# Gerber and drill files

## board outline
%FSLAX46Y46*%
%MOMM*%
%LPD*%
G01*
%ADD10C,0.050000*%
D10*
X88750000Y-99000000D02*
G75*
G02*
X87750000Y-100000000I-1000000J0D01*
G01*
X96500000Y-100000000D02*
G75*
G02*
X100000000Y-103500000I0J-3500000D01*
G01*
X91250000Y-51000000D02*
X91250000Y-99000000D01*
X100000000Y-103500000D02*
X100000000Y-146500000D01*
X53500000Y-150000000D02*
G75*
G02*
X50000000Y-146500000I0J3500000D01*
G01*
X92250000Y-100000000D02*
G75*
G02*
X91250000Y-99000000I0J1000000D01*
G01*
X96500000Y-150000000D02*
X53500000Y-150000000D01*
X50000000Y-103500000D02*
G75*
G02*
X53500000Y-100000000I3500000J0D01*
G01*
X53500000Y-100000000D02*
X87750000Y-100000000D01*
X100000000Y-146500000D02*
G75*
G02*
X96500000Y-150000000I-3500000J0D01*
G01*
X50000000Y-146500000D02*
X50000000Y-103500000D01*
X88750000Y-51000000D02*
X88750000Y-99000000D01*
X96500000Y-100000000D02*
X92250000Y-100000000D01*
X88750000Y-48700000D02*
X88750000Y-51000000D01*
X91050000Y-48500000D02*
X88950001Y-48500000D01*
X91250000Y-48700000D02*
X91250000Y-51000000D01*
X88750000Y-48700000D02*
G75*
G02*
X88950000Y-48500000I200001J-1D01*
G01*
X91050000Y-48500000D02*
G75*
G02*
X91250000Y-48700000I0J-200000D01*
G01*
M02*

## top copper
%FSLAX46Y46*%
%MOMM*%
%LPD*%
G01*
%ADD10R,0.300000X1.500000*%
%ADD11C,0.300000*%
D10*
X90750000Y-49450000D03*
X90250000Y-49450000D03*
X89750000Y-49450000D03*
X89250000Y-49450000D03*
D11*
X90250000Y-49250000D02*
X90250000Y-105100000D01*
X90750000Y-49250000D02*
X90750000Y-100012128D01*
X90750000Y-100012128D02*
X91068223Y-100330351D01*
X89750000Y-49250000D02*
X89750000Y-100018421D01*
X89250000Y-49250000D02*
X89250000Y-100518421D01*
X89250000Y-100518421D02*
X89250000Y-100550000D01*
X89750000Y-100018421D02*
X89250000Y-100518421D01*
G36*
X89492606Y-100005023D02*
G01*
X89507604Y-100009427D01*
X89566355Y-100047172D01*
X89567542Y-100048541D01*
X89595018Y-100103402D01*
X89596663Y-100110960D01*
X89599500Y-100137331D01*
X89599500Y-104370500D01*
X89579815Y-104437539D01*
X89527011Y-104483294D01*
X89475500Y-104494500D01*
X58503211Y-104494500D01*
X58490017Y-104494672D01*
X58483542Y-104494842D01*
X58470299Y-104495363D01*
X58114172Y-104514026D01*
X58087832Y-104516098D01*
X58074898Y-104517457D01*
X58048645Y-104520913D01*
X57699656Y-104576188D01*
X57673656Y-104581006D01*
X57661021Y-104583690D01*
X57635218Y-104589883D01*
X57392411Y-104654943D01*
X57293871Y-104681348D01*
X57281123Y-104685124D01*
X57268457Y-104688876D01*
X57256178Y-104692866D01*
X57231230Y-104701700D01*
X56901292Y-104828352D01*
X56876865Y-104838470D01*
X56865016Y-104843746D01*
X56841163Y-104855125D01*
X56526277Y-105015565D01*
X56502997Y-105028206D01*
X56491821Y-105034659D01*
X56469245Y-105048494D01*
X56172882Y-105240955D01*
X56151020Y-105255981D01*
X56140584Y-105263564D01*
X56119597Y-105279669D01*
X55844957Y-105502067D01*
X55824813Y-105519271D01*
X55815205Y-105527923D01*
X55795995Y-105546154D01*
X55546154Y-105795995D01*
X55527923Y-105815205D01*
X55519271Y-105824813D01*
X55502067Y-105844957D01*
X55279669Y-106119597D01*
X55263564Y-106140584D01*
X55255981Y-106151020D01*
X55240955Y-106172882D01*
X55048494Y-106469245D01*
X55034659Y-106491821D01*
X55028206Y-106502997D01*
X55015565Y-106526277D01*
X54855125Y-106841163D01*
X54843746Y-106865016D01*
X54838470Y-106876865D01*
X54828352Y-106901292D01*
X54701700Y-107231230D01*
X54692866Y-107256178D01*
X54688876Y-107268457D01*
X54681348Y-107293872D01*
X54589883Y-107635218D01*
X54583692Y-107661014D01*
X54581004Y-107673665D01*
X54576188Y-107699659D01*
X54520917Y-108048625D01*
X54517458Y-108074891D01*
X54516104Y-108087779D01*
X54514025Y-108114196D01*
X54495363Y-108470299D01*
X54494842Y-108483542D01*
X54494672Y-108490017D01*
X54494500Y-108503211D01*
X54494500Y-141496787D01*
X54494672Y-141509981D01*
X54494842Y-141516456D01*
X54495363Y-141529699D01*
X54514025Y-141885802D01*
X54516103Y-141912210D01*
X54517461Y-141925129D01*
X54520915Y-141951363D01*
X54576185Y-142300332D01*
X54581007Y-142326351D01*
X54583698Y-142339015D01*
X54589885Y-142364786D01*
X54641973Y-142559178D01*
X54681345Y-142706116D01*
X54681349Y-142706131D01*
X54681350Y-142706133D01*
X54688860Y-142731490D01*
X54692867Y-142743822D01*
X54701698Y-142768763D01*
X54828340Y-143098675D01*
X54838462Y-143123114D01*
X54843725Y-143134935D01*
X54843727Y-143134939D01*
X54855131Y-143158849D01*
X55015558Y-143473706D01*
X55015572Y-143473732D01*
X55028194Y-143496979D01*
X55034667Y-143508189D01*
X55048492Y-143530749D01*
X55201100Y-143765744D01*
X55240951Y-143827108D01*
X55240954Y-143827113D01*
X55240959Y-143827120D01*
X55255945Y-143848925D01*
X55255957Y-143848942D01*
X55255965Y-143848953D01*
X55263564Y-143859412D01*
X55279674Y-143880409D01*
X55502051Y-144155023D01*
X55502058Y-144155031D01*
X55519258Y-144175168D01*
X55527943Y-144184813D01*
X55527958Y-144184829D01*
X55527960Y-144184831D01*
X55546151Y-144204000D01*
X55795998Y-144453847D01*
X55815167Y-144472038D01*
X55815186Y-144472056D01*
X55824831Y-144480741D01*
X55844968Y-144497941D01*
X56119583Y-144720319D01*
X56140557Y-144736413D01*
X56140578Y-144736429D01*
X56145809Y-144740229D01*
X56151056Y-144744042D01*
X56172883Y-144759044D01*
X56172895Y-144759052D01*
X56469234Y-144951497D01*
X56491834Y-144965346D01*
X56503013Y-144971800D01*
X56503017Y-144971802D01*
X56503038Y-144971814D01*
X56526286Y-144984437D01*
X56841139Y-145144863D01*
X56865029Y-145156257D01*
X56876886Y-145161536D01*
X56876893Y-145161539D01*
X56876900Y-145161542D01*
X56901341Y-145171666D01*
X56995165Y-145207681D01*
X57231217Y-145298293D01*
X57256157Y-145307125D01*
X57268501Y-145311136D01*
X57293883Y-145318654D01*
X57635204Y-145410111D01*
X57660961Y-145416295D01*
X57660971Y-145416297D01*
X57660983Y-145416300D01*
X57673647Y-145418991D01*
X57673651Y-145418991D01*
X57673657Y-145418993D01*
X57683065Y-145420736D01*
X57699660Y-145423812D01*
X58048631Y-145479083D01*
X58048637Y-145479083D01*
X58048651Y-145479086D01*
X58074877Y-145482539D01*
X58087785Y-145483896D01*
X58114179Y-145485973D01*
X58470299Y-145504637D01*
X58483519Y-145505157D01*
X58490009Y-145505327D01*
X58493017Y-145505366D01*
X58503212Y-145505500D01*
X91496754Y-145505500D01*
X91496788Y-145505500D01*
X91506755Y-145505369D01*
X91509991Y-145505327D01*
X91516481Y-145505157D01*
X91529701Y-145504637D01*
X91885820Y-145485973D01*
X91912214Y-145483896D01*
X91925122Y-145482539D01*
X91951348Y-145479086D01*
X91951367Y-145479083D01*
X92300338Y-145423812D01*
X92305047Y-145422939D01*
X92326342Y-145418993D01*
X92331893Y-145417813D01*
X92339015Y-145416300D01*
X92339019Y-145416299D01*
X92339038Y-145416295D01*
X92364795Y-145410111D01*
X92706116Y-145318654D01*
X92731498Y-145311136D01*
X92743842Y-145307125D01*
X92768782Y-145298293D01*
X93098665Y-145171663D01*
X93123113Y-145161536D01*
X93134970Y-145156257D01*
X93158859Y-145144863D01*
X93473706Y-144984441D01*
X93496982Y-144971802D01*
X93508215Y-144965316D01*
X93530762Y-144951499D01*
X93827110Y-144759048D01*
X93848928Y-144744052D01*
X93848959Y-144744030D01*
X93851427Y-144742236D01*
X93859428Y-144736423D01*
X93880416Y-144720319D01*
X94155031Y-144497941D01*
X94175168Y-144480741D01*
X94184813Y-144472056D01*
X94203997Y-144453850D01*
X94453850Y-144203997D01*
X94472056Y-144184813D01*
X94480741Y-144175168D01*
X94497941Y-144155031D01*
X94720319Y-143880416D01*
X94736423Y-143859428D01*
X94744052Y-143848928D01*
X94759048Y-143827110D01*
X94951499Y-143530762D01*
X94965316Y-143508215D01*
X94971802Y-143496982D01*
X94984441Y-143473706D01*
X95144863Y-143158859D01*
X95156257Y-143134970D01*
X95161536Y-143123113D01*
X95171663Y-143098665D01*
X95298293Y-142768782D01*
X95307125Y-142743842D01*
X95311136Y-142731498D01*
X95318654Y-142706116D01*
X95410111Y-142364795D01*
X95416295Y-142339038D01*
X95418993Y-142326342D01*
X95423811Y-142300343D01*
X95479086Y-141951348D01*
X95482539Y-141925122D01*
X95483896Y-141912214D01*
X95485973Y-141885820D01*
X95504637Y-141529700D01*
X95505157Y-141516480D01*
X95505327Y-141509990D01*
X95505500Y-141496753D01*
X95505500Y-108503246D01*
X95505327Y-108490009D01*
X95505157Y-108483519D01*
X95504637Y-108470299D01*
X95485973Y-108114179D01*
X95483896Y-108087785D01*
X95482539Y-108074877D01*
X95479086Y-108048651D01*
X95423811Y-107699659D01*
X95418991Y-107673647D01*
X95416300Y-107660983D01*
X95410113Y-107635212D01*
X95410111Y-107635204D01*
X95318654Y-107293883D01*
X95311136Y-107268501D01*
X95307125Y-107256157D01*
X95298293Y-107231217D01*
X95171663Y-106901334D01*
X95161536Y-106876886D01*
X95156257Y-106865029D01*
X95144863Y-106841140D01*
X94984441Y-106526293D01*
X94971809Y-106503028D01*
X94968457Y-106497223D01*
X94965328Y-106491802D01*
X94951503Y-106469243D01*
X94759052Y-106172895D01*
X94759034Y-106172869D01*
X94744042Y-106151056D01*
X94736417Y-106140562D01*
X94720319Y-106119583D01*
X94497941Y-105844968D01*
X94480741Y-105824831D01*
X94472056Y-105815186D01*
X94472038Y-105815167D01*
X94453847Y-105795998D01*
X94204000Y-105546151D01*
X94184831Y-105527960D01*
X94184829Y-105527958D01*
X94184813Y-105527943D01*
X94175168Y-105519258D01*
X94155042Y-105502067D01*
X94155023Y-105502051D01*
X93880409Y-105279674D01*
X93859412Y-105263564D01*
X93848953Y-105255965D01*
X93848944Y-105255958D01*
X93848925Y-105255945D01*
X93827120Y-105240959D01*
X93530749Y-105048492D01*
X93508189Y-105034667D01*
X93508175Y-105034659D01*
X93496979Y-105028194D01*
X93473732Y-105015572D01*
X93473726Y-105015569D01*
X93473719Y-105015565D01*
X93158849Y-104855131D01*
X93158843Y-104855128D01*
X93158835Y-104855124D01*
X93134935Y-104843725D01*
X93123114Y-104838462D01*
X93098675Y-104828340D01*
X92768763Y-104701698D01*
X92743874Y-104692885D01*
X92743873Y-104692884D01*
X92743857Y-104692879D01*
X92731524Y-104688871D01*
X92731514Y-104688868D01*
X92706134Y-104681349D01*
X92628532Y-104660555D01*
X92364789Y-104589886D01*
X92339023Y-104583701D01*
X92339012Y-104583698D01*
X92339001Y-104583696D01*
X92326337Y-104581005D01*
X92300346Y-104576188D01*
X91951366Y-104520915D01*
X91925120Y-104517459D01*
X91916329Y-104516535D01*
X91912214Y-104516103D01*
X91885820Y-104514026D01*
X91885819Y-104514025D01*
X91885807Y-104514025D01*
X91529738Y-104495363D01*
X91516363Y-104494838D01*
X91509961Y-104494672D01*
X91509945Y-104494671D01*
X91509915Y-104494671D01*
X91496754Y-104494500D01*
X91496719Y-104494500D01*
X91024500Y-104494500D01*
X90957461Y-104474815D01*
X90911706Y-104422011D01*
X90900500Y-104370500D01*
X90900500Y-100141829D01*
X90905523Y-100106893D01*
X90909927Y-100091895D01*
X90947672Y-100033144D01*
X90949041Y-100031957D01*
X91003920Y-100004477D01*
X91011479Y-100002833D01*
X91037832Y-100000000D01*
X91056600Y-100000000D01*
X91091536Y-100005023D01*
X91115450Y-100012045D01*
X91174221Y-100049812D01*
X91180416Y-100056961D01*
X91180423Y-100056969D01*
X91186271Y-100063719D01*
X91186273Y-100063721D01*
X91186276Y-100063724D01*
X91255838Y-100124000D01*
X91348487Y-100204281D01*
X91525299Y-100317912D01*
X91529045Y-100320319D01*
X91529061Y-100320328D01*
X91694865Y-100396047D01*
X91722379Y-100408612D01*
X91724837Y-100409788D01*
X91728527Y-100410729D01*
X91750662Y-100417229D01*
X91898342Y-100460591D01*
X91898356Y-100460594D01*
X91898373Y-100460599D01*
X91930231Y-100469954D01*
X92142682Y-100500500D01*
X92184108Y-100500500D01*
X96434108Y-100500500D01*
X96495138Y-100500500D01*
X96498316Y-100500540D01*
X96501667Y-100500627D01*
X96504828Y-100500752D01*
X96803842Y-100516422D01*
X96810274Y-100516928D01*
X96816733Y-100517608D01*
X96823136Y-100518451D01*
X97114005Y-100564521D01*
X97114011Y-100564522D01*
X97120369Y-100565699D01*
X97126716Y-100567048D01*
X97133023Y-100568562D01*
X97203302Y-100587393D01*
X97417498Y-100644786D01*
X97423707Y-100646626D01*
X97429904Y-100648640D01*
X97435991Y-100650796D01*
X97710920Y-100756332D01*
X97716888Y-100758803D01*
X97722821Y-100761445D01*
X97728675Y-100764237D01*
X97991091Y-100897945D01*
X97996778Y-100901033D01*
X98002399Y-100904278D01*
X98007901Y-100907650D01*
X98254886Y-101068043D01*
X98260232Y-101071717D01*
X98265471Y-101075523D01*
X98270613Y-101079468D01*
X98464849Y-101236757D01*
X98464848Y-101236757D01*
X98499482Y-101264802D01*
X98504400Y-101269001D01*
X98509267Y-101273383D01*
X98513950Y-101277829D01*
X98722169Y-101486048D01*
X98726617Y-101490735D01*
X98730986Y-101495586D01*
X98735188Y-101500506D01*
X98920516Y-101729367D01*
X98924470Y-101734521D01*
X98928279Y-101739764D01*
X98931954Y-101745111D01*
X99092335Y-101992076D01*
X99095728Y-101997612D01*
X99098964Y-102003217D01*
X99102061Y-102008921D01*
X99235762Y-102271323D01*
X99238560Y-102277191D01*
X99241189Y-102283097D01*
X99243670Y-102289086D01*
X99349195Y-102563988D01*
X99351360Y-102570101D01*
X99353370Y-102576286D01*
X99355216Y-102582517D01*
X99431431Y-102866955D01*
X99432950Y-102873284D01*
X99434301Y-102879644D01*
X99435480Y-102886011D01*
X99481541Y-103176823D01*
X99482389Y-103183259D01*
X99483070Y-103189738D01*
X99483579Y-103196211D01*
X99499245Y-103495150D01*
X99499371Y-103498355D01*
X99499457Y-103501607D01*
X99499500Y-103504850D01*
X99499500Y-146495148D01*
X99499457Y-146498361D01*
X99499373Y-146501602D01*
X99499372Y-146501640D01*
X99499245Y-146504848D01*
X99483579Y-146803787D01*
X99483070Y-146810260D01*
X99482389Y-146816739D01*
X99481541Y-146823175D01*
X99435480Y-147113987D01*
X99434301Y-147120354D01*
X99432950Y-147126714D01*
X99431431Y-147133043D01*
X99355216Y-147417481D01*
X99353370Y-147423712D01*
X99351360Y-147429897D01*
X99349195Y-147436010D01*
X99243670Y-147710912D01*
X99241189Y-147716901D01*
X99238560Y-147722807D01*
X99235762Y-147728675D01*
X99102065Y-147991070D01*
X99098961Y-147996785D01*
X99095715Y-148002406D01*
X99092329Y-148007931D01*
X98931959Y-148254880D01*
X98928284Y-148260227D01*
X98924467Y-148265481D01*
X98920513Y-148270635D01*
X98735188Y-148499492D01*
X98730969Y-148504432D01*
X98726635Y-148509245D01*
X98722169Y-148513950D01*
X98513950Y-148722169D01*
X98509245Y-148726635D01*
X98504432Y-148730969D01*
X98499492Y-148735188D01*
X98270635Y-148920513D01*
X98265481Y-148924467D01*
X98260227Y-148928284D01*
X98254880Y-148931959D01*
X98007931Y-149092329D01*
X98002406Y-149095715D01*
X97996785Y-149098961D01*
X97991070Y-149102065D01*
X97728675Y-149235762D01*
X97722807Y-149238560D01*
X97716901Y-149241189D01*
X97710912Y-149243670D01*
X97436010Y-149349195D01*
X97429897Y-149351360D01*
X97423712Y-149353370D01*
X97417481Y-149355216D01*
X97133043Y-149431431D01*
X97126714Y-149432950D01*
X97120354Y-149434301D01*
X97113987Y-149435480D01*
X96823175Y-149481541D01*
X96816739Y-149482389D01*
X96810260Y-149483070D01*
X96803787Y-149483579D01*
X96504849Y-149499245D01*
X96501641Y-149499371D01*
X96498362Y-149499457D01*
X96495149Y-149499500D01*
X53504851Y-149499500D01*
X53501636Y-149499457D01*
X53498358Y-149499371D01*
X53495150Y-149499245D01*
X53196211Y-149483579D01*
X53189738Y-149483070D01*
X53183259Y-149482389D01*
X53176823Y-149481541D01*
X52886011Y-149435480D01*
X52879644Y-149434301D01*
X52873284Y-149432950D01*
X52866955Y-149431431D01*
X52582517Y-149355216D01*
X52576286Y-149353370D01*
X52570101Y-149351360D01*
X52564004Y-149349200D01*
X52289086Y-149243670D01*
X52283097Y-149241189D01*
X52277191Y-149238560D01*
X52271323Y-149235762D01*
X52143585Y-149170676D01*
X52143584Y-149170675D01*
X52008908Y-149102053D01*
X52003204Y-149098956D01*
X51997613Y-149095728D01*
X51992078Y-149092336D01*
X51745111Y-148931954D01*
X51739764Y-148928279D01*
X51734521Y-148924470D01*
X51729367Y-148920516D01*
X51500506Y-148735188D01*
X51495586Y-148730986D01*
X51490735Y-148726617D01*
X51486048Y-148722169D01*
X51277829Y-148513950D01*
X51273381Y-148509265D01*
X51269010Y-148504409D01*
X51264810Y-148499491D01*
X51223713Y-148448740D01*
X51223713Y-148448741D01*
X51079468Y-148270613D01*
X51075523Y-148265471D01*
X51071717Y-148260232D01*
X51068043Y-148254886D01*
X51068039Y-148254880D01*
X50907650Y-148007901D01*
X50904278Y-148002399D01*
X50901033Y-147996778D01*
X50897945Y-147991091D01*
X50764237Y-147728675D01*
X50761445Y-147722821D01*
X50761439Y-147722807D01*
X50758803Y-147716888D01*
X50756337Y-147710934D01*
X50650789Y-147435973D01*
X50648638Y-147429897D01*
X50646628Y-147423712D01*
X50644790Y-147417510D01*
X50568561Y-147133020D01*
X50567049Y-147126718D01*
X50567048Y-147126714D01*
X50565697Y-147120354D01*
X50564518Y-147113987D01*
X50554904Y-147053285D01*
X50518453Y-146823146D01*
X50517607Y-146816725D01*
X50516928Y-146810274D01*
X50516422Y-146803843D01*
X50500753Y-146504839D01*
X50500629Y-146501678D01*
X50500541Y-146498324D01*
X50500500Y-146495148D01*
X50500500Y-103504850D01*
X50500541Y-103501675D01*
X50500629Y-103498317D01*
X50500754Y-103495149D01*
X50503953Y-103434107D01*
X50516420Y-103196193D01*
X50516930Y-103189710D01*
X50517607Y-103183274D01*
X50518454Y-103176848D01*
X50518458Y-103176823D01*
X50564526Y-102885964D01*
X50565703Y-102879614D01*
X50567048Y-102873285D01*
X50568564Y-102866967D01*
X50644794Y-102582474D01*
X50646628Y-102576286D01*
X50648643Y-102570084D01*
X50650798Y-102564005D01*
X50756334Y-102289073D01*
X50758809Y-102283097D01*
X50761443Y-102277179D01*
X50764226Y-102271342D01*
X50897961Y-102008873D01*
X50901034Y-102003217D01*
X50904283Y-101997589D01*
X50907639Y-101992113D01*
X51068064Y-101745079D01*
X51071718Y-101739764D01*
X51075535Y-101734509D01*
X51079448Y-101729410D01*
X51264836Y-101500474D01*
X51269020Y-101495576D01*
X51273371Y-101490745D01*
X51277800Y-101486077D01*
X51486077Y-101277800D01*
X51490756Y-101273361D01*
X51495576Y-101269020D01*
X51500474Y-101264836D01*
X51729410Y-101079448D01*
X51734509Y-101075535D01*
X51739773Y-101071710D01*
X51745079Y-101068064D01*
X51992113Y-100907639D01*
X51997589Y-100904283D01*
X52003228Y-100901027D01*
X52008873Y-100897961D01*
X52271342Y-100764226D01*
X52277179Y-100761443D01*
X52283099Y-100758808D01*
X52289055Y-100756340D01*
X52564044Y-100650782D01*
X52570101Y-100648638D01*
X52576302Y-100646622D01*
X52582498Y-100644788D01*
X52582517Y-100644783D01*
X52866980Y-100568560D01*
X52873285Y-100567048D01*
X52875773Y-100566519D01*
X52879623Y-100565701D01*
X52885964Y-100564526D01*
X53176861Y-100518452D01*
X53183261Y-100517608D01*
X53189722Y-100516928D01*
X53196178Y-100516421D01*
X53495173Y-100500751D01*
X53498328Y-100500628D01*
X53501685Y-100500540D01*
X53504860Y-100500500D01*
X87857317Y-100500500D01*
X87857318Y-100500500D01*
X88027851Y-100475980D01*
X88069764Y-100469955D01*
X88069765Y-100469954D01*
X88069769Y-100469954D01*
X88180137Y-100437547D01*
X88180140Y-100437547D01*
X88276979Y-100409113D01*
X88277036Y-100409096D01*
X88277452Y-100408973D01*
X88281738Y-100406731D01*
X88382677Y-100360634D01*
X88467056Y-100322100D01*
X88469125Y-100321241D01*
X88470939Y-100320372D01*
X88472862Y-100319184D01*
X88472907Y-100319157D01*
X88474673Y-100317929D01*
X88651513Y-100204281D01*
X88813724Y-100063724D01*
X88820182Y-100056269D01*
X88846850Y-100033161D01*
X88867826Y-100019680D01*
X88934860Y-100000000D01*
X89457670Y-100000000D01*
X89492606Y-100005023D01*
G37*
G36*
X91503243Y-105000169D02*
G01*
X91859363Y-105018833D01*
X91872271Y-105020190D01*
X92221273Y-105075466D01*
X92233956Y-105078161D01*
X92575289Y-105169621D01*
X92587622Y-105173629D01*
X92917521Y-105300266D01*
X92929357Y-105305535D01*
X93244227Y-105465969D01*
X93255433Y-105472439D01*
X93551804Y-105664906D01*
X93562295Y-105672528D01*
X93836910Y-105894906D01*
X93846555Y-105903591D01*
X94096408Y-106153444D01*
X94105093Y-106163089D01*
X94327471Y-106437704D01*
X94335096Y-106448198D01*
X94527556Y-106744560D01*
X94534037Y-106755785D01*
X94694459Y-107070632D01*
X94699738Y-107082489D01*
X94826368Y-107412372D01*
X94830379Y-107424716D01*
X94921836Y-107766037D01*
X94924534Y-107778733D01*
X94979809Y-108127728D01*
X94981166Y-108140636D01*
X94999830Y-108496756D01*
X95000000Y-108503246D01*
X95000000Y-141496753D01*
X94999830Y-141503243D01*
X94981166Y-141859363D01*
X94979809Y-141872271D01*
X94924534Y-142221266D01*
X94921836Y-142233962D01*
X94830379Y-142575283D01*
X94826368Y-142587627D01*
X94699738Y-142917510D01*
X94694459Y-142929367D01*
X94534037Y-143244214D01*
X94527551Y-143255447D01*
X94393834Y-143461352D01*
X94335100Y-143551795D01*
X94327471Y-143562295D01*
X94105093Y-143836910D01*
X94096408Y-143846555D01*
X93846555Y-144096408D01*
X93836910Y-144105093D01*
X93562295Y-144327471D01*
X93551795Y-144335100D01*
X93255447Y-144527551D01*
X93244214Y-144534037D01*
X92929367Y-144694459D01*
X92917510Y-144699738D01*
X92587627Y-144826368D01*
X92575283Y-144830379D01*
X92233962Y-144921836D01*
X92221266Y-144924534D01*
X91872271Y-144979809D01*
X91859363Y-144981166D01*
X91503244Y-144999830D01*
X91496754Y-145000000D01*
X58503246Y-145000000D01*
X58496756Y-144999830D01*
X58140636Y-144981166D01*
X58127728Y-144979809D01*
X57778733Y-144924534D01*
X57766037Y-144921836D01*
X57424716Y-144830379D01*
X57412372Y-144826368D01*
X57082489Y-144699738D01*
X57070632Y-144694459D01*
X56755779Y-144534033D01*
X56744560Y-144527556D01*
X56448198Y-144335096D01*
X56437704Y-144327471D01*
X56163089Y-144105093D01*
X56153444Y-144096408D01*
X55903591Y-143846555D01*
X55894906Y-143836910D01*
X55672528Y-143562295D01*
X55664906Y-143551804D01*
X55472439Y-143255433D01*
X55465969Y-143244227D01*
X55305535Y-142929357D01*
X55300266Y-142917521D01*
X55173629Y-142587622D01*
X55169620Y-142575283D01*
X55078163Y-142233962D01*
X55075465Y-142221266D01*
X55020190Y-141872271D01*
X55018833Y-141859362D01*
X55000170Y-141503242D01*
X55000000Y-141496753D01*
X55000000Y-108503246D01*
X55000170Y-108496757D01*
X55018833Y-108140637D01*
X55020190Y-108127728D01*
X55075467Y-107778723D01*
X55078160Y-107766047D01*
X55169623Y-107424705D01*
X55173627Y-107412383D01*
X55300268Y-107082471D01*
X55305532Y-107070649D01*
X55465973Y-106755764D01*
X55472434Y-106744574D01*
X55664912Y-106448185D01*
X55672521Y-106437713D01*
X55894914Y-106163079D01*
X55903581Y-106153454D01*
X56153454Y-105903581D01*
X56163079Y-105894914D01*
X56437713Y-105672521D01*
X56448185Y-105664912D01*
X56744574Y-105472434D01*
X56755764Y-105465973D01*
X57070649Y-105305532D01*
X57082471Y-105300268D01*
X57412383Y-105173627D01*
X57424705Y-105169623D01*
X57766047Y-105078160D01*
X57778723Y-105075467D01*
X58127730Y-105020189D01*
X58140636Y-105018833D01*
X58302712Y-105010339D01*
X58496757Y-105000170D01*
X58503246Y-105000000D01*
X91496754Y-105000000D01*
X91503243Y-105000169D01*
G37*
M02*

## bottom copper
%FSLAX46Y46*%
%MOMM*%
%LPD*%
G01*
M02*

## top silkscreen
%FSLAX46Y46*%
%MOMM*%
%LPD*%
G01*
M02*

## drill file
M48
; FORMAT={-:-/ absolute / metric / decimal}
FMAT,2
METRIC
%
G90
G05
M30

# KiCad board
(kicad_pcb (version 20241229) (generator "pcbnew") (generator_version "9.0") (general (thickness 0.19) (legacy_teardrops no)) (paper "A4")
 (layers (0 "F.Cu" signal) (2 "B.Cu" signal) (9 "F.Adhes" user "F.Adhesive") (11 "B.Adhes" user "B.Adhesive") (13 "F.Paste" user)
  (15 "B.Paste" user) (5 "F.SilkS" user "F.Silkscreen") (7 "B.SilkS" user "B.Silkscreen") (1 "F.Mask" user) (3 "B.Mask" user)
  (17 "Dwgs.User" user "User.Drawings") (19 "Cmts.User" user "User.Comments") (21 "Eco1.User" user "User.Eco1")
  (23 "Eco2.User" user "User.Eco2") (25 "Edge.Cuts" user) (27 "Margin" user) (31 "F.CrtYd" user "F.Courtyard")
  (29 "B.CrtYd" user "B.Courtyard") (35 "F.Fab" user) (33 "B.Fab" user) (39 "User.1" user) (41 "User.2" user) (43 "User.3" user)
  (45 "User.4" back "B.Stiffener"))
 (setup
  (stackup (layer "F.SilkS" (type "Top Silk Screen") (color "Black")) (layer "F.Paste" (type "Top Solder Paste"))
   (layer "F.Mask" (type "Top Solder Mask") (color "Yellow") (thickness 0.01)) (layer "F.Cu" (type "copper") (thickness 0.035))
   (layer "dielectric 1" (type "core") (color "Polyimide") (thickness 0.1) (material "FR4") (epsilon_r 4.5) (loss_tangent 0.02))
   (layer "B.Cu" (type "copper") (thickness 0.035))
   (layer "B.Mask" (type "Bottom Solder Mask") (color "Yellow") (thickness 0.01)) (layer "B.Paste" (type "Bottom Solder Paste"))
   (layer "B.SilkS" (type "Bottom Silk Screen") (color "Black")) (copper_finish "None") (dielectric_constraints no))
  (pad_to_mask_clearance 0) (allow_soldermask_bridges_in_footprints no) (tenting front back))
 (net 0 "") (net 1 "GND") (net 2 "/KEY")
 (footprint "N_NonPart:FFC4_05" (layer "F.Cu") (at 90 50)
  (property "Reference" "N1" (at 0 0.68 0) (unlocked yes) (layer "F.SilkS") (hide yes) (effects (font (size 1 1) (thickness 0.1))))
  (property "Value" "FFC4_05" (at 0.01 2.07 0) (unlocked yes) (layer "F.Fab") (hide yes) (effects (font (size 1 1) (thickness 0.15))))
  (fp_line (start -1.25 -1.3) (end -1.25 1) (stroke (width 0.05) (type default)) (layer "Edge.Cuts"))
  (fp_line (start 1.05 -1.5) (end -1.049999 -1.5) (stroke (width 0.05) (type default)) (layer "Edge.Cuts"))
  (fp_line (start 1.25 -1.3) (end 1.25 1) (stroke (width 0.05) (type default)) (layer "Edge.Cuts"))
  (fp_arc (start -1.25 -1.3) (mid -1.191421 -1.441421) (end -1.05 -1.5) (stroke (width 0.05) (type default)) (layer "Edge.Cuts"))
  (fp_arc (start 1.05 -1.5) (mid 1.191421 -1.441421) (end 1.25 -1.3) (stroke (width 0.05) (type default)) (layer "Edge.Cuts"))
  (pad "1" smd rect (at 0.75 -0.55) (size 0.3 1.5) (layers "F.Cu") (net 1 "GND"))
  (pad "2" smd rect (at 0.25 -0.55) (size 0.3 1.5) (layers "F.Cu") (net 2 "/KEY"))
  (pad "3" smd rect (at -0.25 -0.55) (size 0.3 1.5) (layers "F.Cu") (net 1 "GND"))
  (pad "4" smd rect (at -0.75 -0.55) (size 0.3 1.5) (layers "F.Cu") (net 1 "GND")))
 (gr_arc (start 88.75 99) (mid 88.457107 99.707107) (end 87.75 100) (stroke (width 0.05) (type default)) (layer "Edge.Cuts"))
 (gr_arc (start 96.5 100) (mid 98.974874 101.025126) (end 100 103.5) (stroke (width 0.05) (type default)) (layer "Edge.Cuts"))
 (gr_line (start 91.25 51) (end 91.25 99) (stroke (width 0.05) (type default)) (layer "Edge.Cuts"))
 (gr_line (start 100 103.5) (end 100 146.5) (stroke (width 0.05) (type default)) (layer "Edge.Cuts"))
 (gr_arc (start 53.5 150) (mid 51.025126 148.974874) (end 50 146.5) (stroke (width 0.05) (type default)) (layer "Edge.Cuts"))
 (gr_arc (start 92.25 100) (mid 91.542893 99.707107) (end 91.25 99) (stroke (width 0.05) (type default)) (layer "Edge.Cuts"))
 (gr_line (start 96.5 150) (end 53.5 150) (stroke (width 0.05) (type default)) (layer "Edge.Cuts"))
 (gr_arc (start 50 103.5) (mid 51.025126 101.025126) (end 53.5 100) (stroke (width 0.05) (type default)) (layer "Edge.Cuts"))
 (gr_line (start 53.5 100) (end 87.75 100) (stroke (width 0.05) (type default)) (layer "Edge.Cuts"))
 (gr_arc (start 100 146.5) (mid 98.974874 148.974874) (end 96.5 150) (stroke (width 0.05) (type default)) (layer "Edge.Cuts"))
 (gr_line (start 50 146.5) (end 50 103.5) (stroke (width 0.05) (type default)) (layer "Edge.Cuts"))
 (gr_line (start 88.75 51) (end 88.75 99) (stroke (width 0.05) (type default)) (layer "Edge.Cuts"))
 (gr_line (start 96.5 100) (end 92.25 100) (stroke (width 0.05) (type default)) (layer "Edge.Cuts"))
 (segment (start 90.25 49.25) (end 90.25 105.1) (width 0.3) (layer "F.Cu") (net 2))
 (segment (start 90.75 49.25) (end 90.75 100.012128) (width 0.3) (layer "F.Cu") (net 1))
 (segment (start 90.75 100.012128) (end 91.068223 100.330351) (width 0.3) (layer "F.Cu") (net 1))
 (segment (start 89.75 49.25) (end 89.75 100.018421) (width 0.3) (layer "F.Cu") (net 1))
 (segment (start 89.25 49.25) (end 89.25 100.518421) (width 0.3) (layer "F.Cu") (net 1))
 (segment (start 89.25 100.518421) (end 89.25 100.55) (width 0.3) (layer "F.Cu") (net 1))
 (segment (start 89.75 100.018421) (end 89.25 100.518421) (width 0.3) (layer "F.Cu") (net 1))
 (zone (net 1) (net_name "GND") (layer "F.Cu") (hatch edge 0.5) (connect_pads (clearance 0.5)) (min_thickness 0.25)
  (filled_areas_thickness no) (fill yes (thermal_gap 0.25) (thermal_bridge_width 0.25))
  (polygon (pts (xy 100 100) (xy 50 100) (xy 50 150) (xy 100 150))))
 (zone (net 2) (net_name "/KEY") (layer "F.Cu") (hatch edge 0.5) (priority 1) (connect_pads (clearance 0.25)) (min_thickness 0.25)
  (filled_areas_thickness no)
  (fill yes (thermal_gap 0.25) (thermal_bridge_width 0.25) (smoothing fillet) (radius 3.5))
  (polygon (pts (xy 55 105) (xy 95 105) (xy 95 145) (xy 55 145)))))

